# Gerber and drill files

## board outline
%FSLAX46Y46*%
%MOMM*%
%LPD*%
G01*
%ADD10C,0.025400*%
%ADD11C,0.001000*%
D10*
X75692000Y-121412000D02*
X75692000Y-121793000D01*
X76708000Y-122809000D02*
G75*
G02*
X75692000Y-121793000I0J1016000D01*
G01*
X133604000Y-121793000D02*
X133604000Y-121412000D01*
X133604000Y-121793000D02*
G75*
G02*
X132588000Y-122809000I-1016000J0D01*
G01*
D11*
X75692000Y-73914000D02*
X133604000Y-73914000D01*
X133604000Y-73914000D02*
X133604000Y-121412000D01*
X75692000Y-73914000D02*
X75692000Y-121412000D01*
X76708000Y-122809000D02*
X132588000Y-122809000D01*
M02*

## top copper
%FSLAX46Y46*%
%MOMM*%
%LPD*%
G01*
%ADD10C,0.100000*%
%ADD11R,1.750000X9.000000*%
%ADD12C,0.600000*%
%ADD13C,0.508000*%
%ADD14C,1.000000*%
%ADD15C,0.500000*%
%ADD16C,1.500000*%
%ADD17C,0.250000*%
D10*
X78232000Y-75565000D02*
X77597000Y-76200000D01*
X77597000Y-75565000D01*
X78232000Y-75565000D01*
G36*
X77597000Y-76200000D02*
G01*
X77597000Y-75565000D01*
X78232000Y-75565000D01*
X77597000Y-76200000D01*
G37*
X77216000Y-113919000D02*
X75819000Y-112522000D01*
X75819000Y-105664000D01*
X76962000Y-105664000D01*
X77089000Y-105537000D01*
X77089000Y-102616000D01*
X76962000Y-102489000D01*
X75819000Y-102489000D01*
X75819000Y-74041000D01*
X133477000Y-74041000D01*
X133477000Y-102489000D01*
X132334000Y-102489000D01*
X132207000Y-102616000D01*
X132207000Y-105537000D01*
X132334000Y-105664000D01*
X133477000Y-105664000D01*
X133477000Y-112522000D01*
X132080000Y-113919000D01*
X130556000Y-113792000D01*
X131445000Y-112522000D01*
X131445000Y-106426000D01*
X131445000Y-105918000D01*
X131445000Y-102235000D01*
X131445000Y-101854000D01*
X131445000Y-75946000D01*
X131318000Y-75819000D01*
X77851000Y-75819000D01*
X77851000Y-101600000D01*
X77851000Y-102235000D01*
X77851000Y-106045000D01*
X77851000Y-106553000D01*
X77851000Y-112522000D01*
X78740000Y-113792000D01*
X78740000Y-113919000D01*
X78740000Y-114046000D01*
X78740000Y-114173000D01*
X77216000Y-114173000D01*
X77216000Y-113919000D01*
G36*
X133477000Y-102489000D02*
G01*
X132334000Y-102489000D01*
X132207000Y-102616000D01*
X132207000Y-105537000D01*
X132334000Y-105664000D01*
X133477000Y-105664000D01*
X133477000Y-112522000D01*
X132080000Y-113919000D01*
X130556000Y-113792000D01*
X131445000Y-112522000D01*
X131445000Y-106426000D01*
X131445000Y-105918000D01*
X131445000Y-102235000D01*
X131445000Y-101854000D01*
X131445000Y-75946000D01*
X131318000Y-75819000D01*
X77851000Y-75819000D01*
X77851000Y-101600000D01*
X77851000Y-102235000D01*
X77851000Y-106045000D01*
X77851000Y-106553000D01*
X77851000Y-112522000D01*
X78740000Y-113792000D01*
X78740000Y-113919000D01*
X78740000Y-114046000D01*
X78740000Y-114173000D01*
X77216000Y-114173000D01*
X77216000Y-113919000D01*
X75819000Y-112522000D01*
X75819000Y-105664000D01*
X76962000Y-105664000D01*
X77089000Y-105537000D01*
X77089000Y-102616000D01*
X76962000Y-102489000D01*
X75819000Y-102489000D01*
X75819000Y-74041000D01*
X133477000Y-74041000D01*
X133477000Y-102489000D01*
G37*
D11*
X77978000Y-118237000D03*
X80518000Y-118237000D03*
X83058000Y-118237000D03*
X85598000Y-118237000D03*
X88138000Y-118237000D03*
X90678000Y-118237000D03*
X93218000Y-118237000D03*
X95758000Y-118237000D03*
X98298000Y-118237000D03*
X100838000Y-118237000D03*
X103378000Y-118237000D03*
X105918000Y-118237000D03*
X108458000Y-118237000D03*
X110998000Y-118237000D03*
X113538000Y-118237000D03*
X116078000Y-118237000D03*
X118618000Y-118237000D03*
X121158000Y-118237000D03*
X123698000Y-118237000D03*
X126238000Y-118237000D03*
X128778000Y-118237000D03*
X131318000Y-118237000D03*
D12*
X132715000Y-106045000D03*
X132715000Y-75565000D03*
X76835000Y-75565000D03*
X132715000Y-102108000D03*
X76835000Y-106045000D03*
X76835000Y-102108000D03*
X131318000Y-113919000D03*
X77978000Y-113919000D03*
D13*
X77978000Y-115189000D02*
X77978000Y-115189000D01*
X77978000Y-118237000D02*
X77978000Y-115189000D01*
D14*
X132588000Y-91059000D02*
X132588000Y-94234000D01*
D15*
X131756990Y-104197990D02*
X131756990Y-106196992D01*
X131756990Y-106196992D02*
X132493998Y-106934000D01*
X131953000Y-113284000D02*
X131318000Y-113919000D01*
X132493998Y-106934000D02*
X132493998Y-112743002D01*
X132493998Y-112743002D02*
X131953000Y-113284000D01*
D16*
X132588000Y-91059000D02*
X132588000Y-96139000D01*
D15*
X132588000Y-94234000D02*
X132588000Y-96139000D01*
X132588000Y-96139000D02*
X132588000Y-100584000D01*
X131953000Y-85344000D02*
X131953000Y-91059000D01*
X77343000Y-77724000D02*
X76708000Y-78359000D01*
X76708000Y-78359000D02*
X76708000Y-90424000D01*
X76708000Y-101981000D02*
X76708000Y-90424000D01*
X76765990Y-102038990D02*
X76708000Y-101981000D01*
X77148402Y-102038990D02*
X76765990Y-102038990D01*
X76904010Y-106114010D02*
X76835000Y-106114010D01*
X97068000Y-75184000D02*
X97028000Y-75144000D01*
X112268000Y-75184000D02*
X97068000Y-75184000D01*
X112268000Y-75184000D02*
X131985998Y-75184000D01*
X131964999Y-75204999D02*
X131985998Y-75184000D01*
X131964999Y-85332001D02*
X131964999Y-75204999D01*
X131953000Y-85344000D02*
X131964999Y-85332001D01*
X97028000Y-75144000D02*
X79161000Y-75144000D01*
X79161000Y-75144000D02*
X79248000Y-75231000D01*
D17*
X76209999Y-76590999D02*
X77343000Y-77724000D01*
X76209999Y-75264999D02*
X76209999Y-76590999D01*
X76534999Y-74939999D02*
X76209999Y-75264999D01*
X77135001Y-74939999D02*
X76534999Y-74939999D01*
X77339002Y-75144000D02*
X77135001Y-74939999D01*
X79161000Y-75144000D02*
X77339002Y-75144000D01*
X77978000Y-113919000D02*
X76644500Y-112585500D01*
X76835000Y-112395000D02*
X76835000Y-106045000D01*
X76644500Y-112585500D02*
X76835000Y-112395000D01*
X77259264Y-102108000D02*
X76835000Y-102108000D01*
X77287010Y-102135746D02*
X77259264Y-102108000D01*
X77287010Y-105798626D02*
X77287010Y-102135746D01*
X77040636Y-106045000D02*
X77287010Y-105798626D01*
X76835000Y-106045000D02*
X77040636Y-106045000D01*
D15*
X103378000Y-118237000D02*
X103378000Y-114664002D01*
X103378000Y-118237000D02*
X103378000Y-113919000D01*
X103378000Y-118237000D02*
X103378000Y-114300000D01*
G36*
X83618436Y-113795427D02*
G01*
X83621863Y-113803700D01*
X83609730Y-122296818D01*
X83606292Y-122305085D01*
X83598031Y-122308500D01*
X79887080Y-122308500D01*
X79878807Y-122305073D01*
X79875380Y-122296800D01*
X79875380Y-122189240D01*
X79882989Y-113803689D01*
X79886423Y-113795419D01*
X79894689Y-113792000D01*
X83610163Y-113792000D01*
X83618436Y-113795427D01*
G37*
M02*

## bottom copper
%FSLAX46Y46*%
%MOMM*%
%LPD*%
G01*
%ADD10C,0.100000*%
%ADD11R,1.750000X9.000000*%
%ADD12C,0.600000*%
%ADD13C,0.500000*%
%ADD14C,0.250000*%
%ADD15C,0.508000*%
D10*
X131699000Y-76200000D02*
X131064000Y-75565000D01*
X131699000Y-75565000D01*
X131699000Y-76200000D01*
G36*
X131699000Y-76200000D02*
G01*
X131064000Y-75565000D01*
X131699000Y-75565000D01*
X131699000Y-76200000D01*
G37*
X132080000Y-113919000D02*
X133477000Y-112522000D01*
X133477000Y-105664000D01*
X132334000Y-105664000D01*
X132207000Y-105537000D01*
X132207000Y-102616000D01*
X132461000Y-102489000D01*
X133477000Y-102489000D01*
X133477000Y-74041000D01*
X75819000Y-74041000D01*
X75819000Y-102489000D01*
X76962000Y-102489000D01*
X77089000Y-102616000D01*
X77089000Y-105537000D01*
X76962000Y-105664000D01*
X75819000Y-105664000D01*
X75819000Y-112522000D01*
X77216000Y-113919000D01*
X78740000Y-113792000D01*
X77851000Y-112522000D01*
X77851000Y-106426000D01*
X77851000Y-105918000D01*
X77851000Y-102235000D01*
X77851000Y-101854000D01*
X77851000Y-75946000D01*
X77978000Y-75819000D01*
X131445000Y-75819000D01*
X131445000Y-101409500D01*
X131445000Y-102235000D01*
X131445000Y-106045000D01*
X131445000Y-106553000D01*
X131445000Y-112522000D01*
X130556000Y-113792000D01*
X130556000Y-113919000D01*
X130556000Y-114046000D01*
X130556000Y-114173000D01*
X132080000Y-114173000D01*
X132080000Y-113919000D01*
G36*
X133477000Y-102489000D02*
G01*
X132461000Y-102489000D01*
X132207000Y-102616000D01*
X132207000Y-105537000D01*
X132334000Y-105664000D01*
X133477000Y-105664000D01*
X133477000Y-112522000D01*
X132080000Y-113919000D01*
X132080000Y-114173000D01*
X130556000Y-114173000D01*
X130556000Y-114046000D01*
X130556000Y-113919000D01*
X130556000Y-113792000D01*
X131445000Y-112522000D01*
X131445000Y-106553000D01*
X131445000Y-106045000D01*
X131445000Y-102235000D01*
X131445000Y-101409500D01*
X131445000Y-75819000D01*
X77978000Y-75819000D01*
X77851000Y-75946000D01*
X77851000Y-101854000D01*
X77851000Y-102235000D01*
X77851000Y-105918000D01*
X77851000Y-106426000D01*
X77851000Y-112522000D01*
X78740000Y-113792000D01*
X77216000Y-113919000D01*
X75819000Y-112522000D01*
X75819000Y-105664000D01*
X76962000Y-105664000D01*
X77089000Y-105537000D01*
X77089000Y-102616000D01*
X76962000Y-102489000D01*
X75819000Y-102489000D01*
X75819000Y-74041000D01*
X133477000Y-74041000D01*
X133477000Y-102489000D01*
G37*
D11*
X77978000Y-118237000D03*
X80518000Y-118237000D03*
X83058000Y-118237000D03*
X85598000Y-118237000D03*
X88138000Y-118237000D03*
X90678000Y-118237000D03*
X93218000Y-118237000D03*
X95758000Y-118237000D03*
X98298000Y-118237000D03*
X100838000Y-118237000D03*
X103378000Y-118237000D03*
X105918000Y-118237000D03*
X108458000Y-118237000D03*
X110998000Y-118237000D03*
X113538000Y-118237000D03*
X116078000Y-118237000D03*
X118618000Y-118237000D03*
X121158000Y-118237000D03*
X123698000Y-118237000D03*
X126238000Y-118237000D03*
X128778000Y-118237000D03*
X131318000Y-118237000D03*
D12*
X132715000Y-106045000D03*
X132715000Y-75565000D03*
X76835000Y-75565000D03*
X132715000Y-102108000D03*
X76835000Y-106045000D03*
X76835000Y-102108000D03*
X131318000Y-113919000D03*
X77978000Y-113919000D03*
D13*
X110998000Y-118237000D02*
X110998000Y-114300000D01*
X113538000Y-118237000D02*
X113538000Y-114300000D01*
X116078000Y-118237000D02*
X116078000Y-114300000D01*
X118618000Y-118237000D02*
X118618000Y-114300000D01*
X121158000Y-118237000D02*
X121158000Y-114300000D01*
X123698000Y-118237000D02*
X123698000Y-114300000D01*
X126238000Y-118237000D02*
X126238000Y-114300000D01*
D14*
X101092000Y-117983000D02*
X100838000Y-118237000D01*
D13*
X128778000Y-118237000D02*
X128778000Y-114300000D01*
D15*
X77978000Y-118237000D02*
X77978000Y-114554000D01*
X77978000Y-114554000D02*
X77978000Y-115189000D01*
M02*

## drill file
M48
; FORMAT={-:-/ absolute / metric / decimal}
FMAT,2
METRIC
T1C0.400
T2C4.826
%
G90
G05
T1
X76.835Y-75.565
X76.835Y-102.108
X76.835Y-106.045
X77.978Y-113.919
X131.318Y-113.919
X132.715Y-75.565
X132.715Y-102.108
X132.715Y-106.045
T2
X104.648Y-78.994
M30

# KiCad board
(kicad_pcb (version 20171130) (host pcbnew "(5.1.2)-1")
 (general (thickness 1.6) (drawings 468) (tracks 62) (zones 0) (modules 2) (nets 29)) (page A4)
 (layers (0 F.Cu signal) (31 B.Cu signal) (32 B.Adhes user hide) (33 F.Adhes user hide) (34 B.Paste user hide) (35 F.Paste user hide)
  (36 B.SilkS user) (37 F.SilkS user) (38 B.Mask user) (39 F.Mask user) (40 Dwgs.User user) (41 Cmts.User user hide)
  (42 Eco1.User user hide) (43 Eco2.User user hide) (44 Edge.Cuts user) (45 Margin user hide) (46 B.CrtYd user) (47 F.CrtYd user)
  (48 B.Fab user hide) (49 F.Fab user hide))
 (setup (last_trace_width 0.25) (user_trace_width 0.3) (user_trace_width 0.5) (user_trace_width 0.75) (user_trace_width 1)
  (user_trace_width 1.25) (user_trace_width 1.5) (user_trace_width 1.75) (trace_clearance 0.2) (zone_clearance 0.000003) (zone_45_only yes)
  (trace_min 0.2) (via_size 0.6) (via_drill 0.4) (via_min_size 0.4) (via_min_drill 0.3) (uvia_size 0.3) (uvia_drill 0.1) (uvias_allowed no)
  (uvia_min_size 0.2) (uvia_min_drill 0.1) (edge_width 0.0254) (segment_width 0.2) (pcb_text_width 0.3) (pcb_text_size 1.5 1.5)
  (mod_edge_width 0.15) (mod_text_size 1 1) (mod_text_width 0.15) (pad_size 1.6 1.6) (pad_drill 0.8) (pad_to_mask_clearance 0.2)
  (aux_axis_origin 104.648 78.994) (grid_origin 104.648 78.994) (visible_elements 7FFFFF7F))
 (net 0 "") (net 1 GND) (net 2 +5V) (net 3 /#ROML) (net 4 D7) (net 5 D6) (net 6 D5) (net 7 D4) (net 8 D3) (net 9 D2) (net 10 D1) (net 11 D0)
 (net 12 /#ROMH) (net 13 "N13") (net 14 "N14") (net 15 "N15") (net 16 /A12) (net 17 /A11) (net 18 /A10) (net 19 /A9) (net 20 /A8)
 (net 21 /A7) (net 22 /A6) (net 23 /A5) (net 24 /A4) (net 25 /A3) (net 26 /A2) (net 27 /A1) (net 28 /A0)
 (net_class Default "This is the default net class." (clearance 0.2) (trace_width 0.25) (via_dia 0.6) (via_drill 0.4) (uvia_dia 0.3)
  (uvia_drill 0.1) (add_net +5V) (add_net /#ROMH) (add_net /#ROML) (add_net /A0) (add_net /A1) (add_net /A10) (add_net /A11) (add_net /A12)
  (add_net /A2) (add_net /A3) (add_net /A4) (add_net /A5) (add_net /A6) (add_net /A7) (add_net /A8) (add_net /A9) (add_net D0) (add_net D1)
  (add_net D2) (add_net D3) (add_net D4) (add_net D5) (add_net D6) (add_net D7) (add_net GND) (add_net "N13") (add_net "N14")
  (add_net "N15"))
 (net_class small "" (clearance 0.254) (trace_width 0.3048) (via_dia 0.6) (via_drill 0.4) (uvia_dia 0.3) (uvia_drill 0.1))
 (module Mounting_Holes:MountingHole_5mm (layer F.Cu) (at 104.648 78.994)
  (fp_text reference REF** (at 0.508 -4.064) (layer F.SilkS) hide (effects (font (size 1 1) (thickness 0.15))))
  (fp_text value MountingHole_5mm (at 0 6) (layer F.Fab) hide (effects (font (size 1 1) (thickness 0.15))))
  (pad "" np_thru_hole circle (at 0 0) (size 4.826 4.826) (drill 4.826) (layers *.Cu)))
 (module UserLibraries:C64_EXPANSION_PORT (layer F.Cu) (at 105.918 118.237)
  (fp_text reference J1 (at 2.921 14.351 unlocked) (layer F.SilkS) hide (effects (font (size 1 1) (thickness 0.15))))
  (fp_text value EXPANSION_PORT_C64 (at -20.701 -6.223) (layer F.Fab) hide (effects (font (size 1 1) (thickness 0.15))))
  (pad 1 connect rect (at -27.94 0) (size 1.75 9) (layers F.Cu F.Mask) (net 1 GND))
  (pad 2 connect rect (at -25.4 0) (size 1.75 9) (layers F.Cu F.Mask) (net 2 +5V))
  (pad 3 connect rect (at -22.86 0) (size 1.75 9) (layers F.Cu F.Mask) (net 2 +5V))
  (pad 4 connect rect (at -20.32 0) (size 1.75 9) (layers F.Cu F.Mask))
  (pad 5 connect rect (at -17.78 0) (size 1.75 9) (layers F.Cu F.Mask))
  (pad 6 connect rect (at -15.24 0) (size 1.75 9) (layers F.Cu F.Mask))
  (pad 7 connect rect (at -12.7 0) (size 1.75 9) (layers F.Cu F.Mask))
  (pad 8 connect rect (at -10.16 0) (size 1.75 9) (layers F.Cu F.Mask) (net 1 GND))
  (pad 9 connect rect (at -7.62 0) (size 1.75 9) (layers F.Cu F.Mask) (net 1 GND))
  (pad 10 connect rect (at -5.08 0) (size 1.75 9) (layers F.Cu F.Mask))
  (pad 11 connect rect (at -2.54 0) (size 1.75 9) (layers F.Cu F.Mask) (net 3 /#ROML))
  (pad 12 connect rect (at 0 0) (size 1.75 9) (layers F.Cu F.Mask))
  (pad 13 connect rect (at 2.54 0) (size 1.75 9) (layers F.Cu F.Mask))
  (pad 14 connect rect (at 5.08 0) (size 1.75 9) (layers F.Cu F.Mask) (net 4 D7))
  (pad 15 connect rect (at 7.62 0) (size 1.75 9) (layers F.Cu F.Mask) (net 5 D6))
  (pad 16 connect rect (at 10.16 0) (size 1.75 9) (layers F.Cu F.Mask) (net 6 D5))
  (pad 17 connect rect (at 12.7 0) (size 1.75 9) (layers F.Cu F.Mask) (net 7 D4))
  (pad 18 connect rect (at 15.24 0) (size 1.75 9) (layers F.Cu F.Mask) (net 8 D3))
  (pad 19 connect rect (at 17.78 0) (size 1.75 9) (layers F.Cu F.Mask) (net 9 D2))
  (pad 20 connect rect (at 20.32 0) (size 1.75 9) (layers F.Cu F.Mask) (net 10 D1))
  (pad 21 connect rect (at 22.86 0) (size 1.75 9) (layers F.Cu F.Mask) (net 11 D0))
  (pad 22 connect rect (at 25.4 0) (size 1.75 9) (layers F.Cu F.Mask) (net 1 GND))
  (pad A connect rect (at -27.94 0) (size 1.75 9) (layers B.Cu F.Mask) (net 1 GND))
  (pad B connect rect (at -25.4 0) (size 1.75 9) (layers B.Cu F.Mask) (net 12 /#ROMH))
  (pad C connect rect (at -22.86 0) (size 1.75 9) (layers B.Cu F.Mask))
  (pad D connect rect (at -20.32 0) (size 1.75 9) (layers B.Cu F.Mask))
  (pad E connect rect (at -17.78 0) (size 1.75 9) (layers B.Cu F.Mask))
  (pad F connect rect (at -15.24 0) (size 1.75 9) (layers B.Cu F.Mask) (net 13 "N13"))
  (pad H connect rect (at -12.7 0) (size 1.75 9) (layers B.Cu F.Mask) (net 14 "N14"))
  (pad J connect rect (at -10.16 0) (size 1.75 9) (layers B.Cu F.Mask) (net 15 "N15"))
  (pad K connect rect (at -7.62 0) (size 1.75 9) (layers B.Cu F.Mask) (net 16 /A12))
  (pad L connect rect (at -5.08 0) (size 1.75 9) (layers B.Cu F.Mask) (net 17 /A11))
  (pad M connect rect (at -2.54 0) (size 1.75 9) (layers B.Cu F.Mask) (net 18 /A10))
  (pad N connect rect (at 0 0) (size 1.75 9) (layers B.Cu F.Mask) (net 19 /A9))
  (pad P connect rect (at 2.54 0) (size 1.75 9) (layers B.Cu F.Mask) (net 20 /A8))
  (pad R connect rect (at 5.08 0) (size 1.75 9) (layers B.Cu F.Mask) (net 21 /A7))
  (pad S connect rect (at 7.62 0) (size 1.75 9) (layers B.Cu F.Mask) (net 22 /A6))
  (pad T connect rect (at 10.16 0) (size 1.75 9) (layers B.Cu F.Mask) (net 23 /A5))
  (pad U connect rect (at 12.7 0) (size 1.75 9) (layers B.Cu F.Mask) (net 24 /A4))
  (pad V connect rect (at 15.24 0) (size 1.75 9) (layers B.Cu F.Mask) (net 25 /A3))
  (pad W connect rect (at 17.78 0) (size 1.75 9) (layers B.Cu F.Mask) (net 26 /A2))
  (pad X connect rect (at 20.32 0) (size 1.75 9) (layers B.Cu F.Mask) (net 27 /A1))
  (pad Y connect rect (at 22.86 0) (size 1.75 9) (layers B.Cu F.Mask) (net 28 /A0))
  (pad Z connect rect (at 25.4 0) (size 1.75 9) (layers B.Cu F.Mask) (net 1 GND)))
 (gr_poly (pts (xy 131.699 76.2) (xy 131.064 75.565) (xy 131.699 75.565)) (layer B.Cu) (width 0.1))
 (gr_poly
  (pts (xy 132.08 113.919) (xy 133.477 112.522) (xy 133.477 105.664) (xy 132.334 105.664) (xy 132.207 105.537) (xy 132.207 102.616)
   (xy 132.461 102.489) (xy 133.477 102.489) (xy 133.477 74.041) (xy 75.819 74.041) (xy 75.819 102.489) (xy 76.962 102.489)
   (xy 77.089 102.616) (xy 77.089 105.537) (xy 76.962 105.664) (xy 75.819 105.664) (xy 75.819 112.522) (xy 77.216 113.919)
   (xy 78.74 113.792) (xy 77.851 112.522) (xy 77.851 106.426) (xy 77.851 105.918) (xy 77.851 102.235) (xy 77.851 101.854) (xy 77.851 75.946)
   (xy 77.978 75.819) (xy 131.445 75.819) (xy 131.445 101.4095) (xy 131.445 102.235) (xy 131.445 106.045) (xy 131.445 106.553)
   (xy 131.445 112.522) (xy 130.556 113.792) (xy 130.556 113.919) (xy 130.556 114.046) (xy 130.556 114.173) (xy 132.08 114.173))
  (layer B.Cu) (width 0.1))
 (gr_poly (pts (xy 78.232 75.565) (xy 77.597 76.2) (xy 77.597 75.565)) (layer F.Cu) (width 0.1))
 (gr_poly
  (pts (xy 77.216 113.919) (xy 75.819 112.522) (xy 75.819 105.664) (xy 76.962 105.664) (xy 77.089 105.537) (xy 77.089 102.616)
   (xy 76.962 102.489) (xy 75.819 102.489) (xy 75.819 74.041) (xy 133.477 74.041) (xy 133.477 102.489) (xy 132.334 102.489)
   (xy 132.207 102.616) (xy 132.207 105.537) (xy 132.334 105.664) (xy 133.477 105.664) (xy 133.477 112.522) (xy 132.08 113.919)
   (xy 130.556 113.792) (xy 131.445 112.522) (xy 131.445 106.426) (xy 131.445 105.918) (xy 131.445 102.235) (xy 131.445 101.854)
   (xy 131.445 75.946) (xy 131.318 75.819) (xy 77.851 75.819) (xy 77.851 101.6) (xy 77.851 102.235) (xy 77.851 106.045) (xy 77.851 106.553)
   (xy 77.851 112.522) (xy 78.74 113.792) (xy 78.74 113.919) (xy 78.74 114.046) (xy 78.74 114.173) (xy 77.216 114.173))
  (layer F.Cu) (width 0.1))
 (gr_line (start 75.692 121.412) (end 75.692 121.793) (angle 90) (layer Edge.Cuts) (width 0.0254))
 (gr_arc (start 76.708 121.793) (end 76.708 122.809) (angle 90) (layer Edge.Cuts) (width 0.0254))
 (gr_line (start 133.604 121.793) (end 133.604 121.412) (angle 90) (layer Edge.Cuts) (width 0.0254))
 (gr_arc (start 132.588 121.793) (end 133.604 121.793) (angle 90) (layer Edge.Cuts) (width 0.0254))
 (gr_line (start 75.692 73.914) (end 133.604 73.914) (angle 90) (layer Edge.Cuts) (width 0.001))
 (gr_line (start 133.604 73.914) (end 133.604 121.412) (angle 90) (layer Edge.Cuts) (width 0.001))
 (gr_line (start 75.692 73.914) (end 75.692 121.412) (angle 90) (layer Edge.Cuts) (width 0.001))
 (gr_line (start 76.708 122.809) (end 132.588 122.809) (angle 90) (layer Edge.Cuts) (width 0.001))
 (via (at 132.715 106.045) (size 0.6) (drill 0.4) (layers F.Cu B.Cu) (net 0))
 (via (at 132.715 75.565) (size 0.6) (drill 0.4) (layers F.Cu B.Cu) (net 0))
 (via (at 76.835 75.565) (size 0.6) (drill 0.4) (layers F.Cu B.Cu) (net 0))
 (via (at 132.715 102.108) (size 0.6) (drill 0.4) (layers F.Cu B.Cu) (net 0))
 (segment (start 110.998 118.237) (end 110.998 114.3) (width 0.5) (layer B.Cu) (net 21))
 (segment (start 113.538 118.237) (end 113.538 114.3) (width 0.5) (layer B.Cu) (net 22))
 (segment (start 116.078 118.237) (end 116.078 114.3) (width 0.5) (layer B.Cu) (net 23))
 (segment (start 118.618 118.237) (end 118.618 114.3) (width 0.5) (layer B.Cu) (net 24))
 (segment (start 121.158 118.237) (end 121.158 114.3) (width 0.5) (layer B.Cu) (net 25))
 (segment (start 123.698 118.237) (end 123.698 114.3) (width 0.5) (layer B.Cu) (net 26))
 (segment (start 126.238 118.237) (end 126.238 114.3) (width 0.5) (layer B.Cu) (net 27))
 (segment (start 101.092 117.983) (end 100.838 118.237) (width 0.25) (layer B.Cu) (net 17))
 (segment (start 128.778 118.237) (end 128.778 114.3) (width 0.5) (layer B.Cu) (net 28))
 (segment (start 77.978 118.237) (end 77.978 114.554) (width 0.508) (layer B.Cu) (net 1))
 (segment (start 77.978 114.554) (end 77.978 115.189) (width 0.508) (layer B.Cu) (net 1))
 (segment (start 77.978 115.189) (end 77.978 115.189) (width 0.508) (layer F.Cu) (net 1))
 (segment (start 77.978 118.237) (end 77.978 115.189) (width 0.508) (layer F.Cu) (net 1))
 (via (at 76.835 106.045) (size 0.6) (drill 0.4) (layers F.Cu B.Cu) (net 1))
 (via (at 76.835 102.108) (size 0.6) (drill 0.4) (layers F.Cu B.Cu) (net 1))
 (via (at 131.318 113.919) (size 0.6) (drill 0.4) (layers F.Cu B.Cu) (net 1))
 (via (at 77.978 113.919) (size 0.6) (drill 0.4) (layers F.Cu B.Cu) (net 1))
 (segment (start 132.588 91.059) (end 132.588 94.234) (width 1) (layer F.Cu) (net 1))
 (segment (start 131.75699 104.19799) (end 131.75699 106.196992) (width 0.5) (layer F.Cu) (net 1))
 (segment (start 131.75699 106.196992) (end 132.493998 106.934) (width 0.5) (layer F.Cu) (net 1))
 (segment (start 131.953 113.284) (end 131.318 113.919) (width 0.5) (layer F.Cu) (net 1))
 (segment (start 132.493998 106.934) (end 132.493998 112.743002) (width 0.5) (layer F.Cu) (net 1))
 (segment (start 132.493998 112.743002) (end 131.953 113.284) (width 0.5) (layer F.Cu) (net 1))
 (segment (start 132.588 91.059) (end 132.588 96.139) (width 1.5) (layer F.Cu) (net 1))
 (segment (start 132.588 94.234) (end 132.588 96.139) (width 0.5) (layer F.Cu) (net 1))
 (segment (start 132.588 96.139) (end 132.588 100.584) (width 0.5) (layer F.Cu) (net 1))
 (segment (start 131.953 85.344) (end 131.953 91.059) (width 0.5) (layer F.Cu) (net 1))
 (segment (start 77.343 77.724) (end 76.708 78.359) (width 0.5) (layer F.Cu) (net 1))
 (segment (start 76.708 78.359) (end 76.708 90.424) (width 0.5) (layer F.Cu) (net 1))
 (segment (start 76.708 101.981) (end 76.708 90.424) (width 0.5) (layer F.Cu) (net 1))
 (segment (start 76.76599 102.03899) (end 76.708 101.981) (width 0.5) (layer F.Cu) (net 1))
 (segment (start 77.148402 102.03899) (end 76.76599 102.03899) (width 0.5) (layer F.Cu) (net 1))
 (segment (start 76.90401 106.11401) (end 76.835 106.11401) (width 0.5) (layer F.Cu) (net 1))
 (segment (start 97.068 75.184) (end 97.028 75.144) (width 0.5) (layer F.Cu) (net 1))
 (segment (start 112.268 75.184) (end 97.068 75.184) (width 0.5) (layer F.Cu) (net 1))
 (segment (start 112.268 75.184) (end 131.985998 75.184) (width 0.5) (layer F.Cu) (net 1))
 (segment (start 131.964999 75.204999) (end 131.985998 75.184) (width 0.5) (layer F.Cu) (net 1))
 (segment (start 131.964999 85.332001) (end 131.964999 75.204999) (width 0.5) (layer F.Cu) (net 1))
 (segment (start 131.953 85.344) (end 131.964999 85.332001) (width 0.5) (layer F.Cu) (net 1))
 (segment (start 97.028 75.144) (end 79.161 75.144) (width 0.5) (layer F.Cu) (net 1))
 (segment (start 79.161 75.144) (end 79.248 75.231) (width 0.5) (layer F.Cu) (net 1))
 (segment (start 76.209999 76.590999) (end 77.343 77.724) (width 0.25) (layer F.Cu) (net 1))
 (segment (start 76.209999 75.264999) (end 76.209999 76.590999) (width 0.25) (layer F.Cu) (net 1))
 (segment (start 76.534999 74.939999) (end 76.209999 75.264999) (width 0.25) (layer F.Cu) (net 1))
 (segment (start 77.135001 74.939999) (end 76.534999 74.939999) (width 0.25) (layer F.Cu) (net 1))
 (segment (start 77.339002 75.144) (end 77.135001 74.939999) (width 0.25) (layer F.Cu) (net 1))
 (segment (start 79.161 75.144) (end 77.339002 75.144) (width 0.25) (layer F.Cu) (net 1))
 (segment (start 77.978 113.919) (end 76.6445 112.5855) (width 0.25) (layer F.Cu) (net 1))
 (segment (start 76.835 112.395) (end 76.835 106.045) (width 0.25) (layer F.Cu) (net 1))
 (segment (start 76.6445 112.5855) (end 76.835 112.395) (width 0.25) (layer F.Cu) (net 1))
 (segment (start 77.259264 102.108) (end 76.835 102.108) (width 0.25) (layer F.Cu) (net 1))
 (segment (start 77.28701 102.135746) (end 77.259264 102.108) (width 0.25) (layer F.Cu) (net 1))
 (segment (start 77.28701 105.798626) (end 77.28701 102.135746) (width 0.25) (layer F.Cu) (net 1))
 (segment (start 77.040636 106.045) (end 77.28701 105.798626) (width 0.25) (layer F.Cu) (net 1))
 (segment (start 76.835 106.045) (end 77.040636 106.045) (width 0.25) (layer F.Cu) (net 1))
 (segment (start 103.378 118.237) (end 103.378 114.664002) (width 0.5) (layer F.Cu) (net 3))
 (segment (start 103.378 118.237) (end 103.378 113.919) (width 0.5) (layer F.Cu) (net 3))
 (segment (start 103.378 118.237) (end 103.378 114.3) (width 0.5) (layer F.Cu) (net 3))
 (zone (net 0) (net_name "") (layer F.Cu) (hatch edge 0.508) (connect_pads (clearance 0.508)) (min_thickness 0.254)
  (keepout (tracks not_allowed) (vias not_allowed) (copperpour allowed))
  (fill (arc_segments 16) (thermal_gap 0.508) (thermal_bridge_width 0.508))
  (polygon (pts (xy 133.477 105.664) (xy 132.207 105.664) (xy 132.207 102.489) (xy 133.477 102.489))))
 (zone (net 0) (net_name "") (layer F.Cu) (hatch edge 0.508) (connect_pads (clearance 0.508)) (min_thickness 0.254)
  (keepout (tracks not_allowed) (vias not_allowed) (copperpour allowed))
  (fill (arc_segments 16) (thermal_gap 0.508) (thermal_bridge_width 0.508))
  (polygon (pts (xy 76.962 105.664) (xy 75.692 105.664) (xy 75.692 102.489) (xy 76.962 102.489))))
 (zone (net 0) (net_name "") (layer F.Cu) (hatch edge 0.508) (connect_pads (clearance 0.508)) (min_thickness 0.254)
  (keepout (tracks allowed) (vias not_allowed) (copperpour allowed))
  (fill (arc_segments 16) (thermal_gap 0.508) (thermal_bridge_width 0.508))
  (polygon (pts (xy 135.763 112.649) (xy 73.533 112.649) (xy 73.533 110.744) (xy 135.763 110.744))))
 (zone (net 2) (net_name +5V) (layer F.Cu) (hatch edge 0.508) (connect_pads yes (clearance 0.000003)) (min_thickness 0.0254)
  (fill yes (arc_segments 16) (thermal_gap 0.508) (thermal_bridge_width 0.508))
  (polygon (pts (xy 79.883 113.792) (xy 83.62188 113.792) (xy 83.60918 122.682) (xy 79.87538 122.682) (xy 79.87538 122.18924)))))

